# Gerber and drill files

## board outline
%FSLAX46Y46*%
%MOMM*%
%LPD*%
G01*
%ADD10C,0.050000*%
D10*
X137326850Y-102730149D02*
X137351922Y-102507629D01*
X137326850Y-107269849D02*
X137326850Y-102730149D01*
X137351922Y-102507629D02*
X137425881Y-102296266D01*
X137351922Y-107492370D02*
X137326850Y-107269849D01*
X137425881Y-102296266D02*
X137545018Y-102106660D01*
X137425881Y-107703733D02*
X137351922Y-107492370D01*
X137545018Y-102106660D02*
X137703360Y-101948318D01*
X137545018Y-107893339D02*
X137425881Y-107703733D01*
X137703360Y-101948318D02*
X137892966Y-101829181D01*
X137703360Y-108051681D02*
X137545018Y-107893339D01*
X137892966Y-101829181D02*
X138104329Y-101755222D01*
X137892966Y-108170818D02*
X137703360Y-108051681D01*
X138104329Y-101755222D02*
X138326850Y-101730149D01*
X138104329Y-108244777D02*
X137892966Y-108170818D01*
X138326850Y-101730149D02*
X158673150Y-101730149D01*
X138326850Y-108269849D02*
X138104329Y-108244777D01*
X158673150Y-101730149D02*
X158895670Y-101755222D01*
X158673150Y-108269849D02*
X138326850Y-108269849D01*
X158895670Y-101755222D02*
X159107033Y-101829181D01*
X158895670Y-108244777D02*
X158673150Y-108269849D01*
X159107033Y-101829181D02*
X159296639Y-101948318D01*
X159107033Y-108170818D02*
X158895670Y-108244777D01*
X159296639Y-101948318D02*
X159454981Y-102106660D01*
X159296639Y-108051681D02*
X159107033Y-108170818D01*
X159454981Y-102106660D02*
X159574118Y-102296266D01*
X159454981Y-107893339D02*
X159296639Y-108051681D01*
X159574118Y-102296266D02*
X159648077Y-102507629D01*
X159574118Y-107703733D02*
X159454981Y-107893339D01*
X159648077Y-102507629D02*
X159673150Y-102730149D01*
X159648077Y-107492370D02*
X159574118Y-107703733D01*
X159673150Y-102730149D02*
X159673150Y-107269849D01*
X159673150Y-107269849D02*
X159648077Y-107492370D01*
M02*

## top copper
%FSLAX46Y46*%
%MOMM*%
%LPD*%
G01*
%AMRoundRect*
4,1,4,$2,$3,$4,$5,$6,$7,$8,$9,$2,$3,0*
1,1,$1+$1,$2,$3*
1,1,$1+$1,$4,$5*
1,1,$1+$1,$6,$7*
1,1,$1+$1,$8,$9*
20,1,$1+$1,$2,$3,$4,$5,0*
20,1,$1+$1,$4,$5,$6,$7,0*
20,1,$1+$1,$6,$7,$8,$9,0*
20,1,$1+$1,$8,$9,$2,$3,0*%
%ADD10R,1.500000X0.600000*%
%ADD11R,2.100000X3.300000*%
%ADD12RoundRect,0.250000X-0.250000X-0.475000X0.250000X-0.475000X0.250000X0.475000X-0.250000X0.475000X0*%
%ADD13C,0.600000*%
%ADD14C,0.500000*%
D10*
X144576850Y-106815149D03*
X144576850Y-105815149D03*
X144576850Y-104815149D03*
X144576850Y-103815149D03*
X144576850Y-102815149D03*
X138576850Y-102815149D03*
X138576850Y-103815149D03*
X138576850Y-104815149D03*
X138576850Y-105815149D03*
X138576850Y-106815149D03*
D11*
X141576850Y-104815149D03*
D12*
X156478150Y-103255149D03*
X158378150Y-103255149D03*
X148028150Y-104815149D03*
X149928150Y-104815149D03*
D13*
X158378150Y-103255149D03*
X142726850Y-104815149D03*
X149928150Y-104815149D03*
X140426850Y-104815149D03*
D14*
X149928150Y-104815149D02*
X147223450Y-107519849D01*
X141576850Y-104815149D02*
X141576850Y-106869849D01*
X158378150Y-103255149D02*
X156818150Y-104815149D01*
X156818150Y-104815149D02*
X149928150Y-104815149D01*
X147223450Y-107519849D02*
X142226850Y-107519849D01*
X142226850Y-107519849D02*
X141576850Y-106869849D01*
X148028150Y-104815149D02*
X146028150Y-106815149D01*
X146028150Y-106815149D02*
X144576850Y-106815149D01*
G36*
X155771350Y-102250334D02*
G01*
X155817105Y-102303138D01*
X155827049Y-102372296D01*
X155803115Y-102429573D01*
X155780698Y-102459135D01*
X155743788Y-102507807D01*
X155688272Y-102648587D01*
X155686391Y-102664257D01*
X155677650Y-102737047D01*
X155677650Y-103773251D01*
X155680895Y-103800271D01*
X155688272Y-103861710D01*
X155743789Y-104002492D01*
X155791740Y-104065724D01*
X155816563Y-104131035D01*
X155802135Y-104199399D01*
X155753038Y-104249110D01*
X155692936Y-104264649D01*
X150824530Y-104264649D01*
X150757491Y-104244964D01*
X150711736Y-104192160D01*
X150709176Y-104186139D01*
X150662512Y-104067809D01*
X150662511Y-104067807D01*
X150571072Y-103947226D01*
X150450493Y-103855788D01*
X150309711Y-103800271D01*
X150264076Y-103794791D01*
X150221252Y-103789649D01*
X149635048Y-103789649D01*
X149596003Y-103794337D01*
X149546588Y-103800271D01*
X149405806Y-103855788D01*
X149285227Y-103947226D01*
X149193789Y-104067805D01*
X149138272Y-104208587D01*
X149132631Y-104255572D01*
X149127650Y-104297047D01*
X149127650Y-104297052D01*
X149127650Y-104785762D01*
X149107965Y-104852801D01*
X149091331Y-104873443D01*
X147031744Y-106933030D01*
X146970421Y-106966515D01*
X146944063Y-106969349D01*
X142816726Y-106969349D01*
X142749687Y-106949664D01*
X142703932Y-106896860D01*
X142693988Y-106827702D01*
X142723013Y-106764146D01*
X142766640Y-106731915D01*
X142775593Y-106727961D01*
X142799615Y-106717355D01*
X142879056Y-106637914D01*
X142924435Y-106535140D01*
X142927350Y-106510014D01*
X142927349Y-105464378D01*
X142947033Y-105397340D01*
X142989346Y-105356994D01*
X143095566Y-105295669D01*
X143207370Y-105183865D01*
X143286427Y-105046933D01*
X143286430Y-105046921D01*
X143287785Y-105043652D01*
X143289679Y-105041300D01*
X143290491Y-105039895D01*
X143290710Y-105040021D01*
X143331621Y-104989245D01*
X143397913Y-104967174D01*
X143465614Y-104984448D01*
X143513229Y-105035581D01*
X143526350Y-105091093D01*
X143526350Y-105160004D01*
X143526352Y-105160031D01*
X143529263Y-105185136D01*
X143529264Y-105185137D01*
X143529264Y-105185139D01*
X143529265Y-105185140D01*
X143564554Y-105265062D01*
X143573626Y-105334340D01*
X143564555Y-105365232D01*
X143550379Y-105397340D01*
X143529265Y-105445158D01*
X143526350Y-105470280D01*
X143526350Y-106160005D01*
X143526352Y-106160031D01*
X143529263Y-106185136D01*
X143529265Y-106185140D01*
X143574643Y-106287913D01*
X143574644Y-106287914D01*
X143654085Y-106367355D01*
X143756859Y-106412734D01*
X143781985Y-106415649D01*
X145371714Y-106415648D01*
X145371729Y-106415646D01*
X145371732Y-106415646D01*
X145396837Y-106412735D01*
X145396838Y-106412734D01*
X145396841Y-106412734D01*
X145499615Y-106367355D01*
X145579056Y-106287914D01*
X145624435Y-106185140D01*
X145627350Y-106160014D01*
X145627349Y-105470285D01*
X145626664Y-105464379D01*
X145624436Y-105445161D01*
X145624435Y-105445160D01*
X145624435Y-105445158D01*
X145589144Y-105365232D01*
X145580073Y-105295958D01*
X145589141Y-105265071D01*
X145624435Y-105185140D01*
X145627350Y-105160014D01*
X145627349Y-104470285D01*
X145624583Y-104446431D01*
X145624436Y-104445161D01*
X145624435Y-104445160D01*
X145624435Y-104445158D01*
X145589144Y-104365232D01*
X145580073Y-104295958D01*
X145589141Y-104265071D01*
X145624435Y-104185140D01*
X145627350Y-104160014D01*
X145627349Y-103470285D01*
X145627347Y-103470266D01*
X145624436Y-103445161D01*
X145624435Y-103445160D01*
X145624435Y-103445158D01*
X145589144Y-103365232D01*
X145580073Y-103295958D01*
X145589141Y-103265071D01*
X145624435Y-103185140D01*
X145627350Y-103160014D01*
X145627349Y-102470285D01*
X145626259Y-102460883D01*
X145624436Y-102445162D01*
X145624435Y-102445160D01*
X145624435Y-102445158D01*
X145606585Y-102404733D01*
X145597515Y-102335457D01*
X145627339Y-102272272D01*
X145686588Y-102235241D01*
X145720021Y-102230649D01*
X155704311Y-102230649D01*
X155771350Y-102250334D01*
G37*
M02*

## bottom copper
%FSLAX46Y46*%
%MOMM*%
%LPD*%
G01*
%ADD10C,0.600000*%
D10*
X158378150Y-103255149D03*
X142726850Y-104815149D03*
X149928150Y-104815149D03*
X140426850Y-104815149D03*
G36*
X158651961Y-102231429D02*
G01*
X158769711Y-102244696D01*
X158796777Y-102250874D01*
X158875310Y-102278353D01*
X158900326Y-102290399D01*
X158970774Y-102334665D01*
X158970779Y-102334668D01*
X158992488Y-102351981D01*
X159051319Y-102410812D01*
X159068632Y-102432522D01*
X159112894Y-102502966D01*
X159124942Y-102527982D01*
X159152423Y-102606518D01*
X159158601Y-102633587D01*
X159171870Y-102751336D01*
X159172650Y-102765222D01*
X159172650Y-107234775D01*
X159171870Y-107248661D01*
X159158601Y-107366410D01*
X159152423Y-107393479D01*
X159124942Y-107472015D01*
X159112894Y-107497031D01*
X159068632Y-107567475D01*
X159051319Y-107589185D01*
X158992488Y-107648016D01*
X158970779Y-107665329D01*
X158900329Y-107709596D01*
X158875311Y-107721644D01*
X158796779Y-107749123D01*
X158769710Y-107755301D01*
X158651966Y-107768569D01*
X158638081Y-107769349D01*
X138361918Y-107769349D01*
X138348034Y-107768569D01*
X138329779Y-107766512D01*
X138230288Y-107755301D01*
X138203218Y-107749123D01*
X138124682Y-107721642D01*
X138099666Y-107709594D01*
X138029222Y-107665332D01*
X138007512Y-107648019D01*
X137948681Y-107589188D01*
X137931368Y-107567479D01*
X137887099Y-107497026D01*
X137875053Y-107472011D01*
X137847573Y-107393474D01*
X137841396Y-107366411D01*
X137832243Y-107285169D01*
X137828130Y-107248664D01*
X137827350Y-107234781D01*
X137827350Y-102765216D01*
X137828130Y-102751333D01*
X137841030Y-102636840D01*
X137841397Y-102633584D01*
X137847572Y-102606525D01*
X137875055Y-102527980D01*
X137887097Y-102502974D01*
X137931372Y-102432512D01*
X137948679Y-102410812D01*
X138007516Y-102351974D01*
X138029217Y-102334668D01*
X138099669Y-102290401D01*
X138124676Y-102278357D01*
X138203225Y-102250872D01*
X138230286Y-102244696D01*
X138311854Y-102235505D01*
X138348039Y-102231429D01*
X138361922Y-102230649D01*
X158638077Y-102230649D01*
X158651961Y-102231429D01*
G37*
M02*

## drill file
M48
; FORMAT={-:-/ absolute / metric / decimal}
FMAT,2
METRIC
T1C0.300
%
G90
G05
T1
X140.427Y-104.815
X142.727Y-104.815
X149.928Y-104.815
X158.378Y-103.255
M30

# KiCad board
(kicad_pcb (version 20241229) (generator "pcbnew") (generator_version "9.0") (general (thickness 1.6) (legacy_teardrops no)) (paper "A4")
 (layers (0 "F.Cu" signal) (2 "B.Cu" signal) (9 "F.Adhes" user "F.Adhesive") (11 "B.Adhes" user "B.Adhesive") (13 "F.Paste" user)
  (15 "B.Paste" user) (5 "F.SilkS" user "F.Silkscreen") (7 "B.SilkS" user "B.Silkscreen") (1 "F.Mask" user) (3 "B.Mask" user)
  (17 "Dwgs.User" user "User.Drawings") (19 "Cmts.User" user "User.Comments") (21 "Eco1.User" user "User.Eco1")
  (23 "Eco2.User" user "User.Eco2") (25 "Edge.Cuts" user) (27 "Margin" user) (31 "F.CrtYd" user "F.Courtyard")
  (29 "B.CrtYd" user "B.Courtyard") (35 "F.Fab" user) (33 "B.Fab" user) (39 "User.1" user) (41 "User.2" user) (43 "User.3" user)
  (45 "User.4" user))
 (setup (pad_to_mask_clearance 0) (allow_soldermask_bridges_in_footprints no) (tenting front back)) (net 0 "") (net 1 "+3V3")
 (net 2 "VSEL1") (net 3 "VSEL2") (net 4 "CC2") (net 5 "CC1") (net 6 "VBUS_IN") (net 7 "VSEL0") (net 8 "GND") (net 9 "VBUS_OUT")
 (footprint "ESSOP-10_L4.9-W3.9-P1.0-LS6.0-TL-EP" (layer "F.Cu") (at 141.57685 104.815149 90)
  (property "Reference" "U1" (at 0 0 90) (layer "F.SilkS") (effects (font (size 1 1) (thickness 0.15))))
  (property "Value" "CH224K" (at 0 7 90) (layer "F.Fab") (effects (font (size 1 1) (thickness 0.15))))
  (pad "1" smd rect (at -2 3 180) (size 1.5 0.6) (layers "F.Cu" "F.Mask" "F.Paste") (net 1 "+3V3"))
  (pad "2" smd rect (at -1 3 180) (size 1.5 0.6) (layers "F.Cu" "F.Mask" "F.Paste") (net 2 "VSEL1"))
  (pad "3" smd rect (at 0 3 180) (size 1.5 0.6) (layers "F.Cu" "F.Mask" "F.Paste") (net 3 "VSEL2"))
  (pad "4" smd rect (at 1 3 180) (size 1.5 0.6) (layers "F.Cu" "F.Mask" "F.Paste"))
  (pad "5" smd rect (at 2 3 180) (size 1.5 0.6) (layers "F.Cu" "F.Mask" "F.Paste"))
  (pad "6" smd rect (at 2 -3 180) (size 1.5 0.6) (layers "F.Cu" "F.Mask" "F.Paste") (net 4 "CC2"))
  (pad "7" smd rect (at 1 -3 180) (size 1.5 0.6) (layers "F.Cu" "F.Mask" "F.Paste") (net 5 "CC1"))
  (pad "8" smd rect (at 0 -3 180) (size 1.5 0.6) (layers "F.Cu" "F.Mask" "F.Paste") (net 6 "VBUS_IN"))
  (pad "9" smd rect (at -1 -3 180) (size 1.5 0.6) (layers "F.Cu" "F.Mask" "F.Paste") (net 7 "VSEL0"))
  (pad "10" smd rect (at -2 -3 180) (size 1.5 0.6) (layers "F.Cu" "F.Mask" "F.Paste"))
  (pad "11" smd rect (at 0 0 270) (size 3.3 2.1) (layers "F.Cu" "F.Mask" "F.Paste") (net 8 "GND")))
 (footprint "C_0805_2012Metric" (layer "F.Cu") (at 157.42815 103.255149)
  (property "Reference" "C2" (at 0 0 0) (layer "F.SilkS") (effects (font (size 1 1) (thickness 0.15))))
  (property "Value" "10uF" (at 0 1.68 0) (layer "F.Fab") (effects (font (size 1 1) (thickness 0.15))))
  (pad "1" smd roundrect (at -0.95 0) (size 1 1.45) (layers "F.Cu" "F.Mask" "F.Paste") (roundrect_rratio 0.25) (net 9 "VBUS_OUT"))
  (pad "2" smd roundrect (at 0.95 0) (size 1 1.45) (layers "F.Cu" "F.Mask" "F.Paste") (roundrect_rratio 0.25) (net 8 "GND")))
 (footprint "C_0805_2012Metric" (layer "F.Cu") (at 148.97815 104.815149)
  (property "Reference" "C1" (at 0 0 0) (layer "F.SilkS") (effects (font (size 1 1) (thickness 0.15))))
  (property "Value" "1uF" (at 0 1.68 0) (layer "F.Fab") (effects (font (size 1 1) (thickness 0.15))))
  (pad "1" smd roundrect (at -0.95 0) (size 1 1.45) (layers "F.Cu" "F.Mask" "F.Paste") (roundrect_rratio 0.25) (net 1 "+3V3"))
  (pad "2" smd roundrect (at 0.95 0) (size 1 1.45) (layers "F.Cu" "F.Mask" "F.Paste") (roundrect_rratio 0.25) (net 8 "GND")))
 (gr_line (start 137.32685 102.730149) (end 137.351922 102.507629) (stroke (width 0.05) (type default)) (layer "Edge.Cuts"))
 (gr_line (start 137.32685 107.269849) (end 137.32685 102.730149) (stroke (width 0.05) (type default)) (layer "Edge.Cuts"))
 (gr_line (start 137.351922 102.507629) (end 137.425881 102.296266) (stroke (width 0.05) (type default)) (layer "Edge.Cuts"))
 (gr_line (start 137.351922 107.49237) (end 137.32685 107.269849) (stroke (width 0.05) (type default)) (layer "Edge.Cuts"))
 (gr_line (start 137.425881 102.296266) (end 137.545018 102.10666) (stroke (width 0.05) (type default)) (layer "Edge.Cuts"))
 (gr_line (start 137.425881 107.703733) (end 137.351922 107.49237) (stroke (width 0.05) (type default)) (layer "Edge.Cuts"))
 (gr_line (start 137.545018 102.10666) (end 137.70336 101.948318) (stroke (width 0.05) (type default)) (layer "Edge.Cuts"))
 (gr_line (start 137.545018 107.893339) (end 137.425881 107.703733) (stroke (width 0.05) (type default)) (layer "Edge.Cuts"))
 (gr_line (start 137.70336 101.948318) (end 137.892966 101.829181) (stroke (width 0.05) (type default)) (layer "Edge.Cuts"))
 (gr_line (start 137.70336 108.051681) (end 137.545018 107.893339) (stroke (width 0.05) (type default)) (layer "Edge.Cuts"))
 (gr_line (start 137.892966 101.829181) (end 138.104329 101.755222) (stroke (width 0.05) (type default)) (layer "Edge.Cuts"))
 (gr_line (start 137.892966 108.170818) (end 137.70336 108.051681) (stroke (width 0.05) (type default)) (layer "Edge.Cuts"))
 (gr_line (start 138.104329 101.755222) (end 138.32685 101.730149) (stroke (width 0.05) (type default)) (layer "Edge.Cuts"))
 (gr_line (start 138.104329 108.244777) (end 137.892966 108.170818) (stroke (width 0.05) (type default)) (layer "Edge.Cuts"))
 (gr_line (start 138.32685 101.730149) (end 158.67315 101.730149) (stroke (width 0.05) (type default)) (layer "Edge.Cuts"))
 (gr_line (start 138.32685 108.269849) (end 138.104329 108.244777) (stroke (width 0.05) (type default)) (layer "Edge.Cuts"))
 (gr_line (start 158.67315 101.730149) (end 158.89567 101.755222) (stroke (width 0.05) (type default)) (layer "Edge.Cuts"))
 (gr_line (start 158.67315 108.269849) (end 138.32685 108.269849) (stroke (width 0.05) (type default)) (layer "Edge.Cuts"))
 (gr_line (start 158.89567 101.755222) (end 159.107033 101.829181) (stroke (width 0.05) (type default)) (layer "Edge.Cuts"))
 (gr_line (start 158.89567 108.244777) (end 158.67315 108.269849) (stroke (width 0.05) (type default)) (layer "Edge.Cuts"))
 (gr_line (start 159.107033 101.829181) (end 159.296639 101.948318) (stroke (width 0.05) (type default)) (layer "Edge.Cuts"))
 (gr_line (start 159.107033 108.170818) (end 158.89567 108.244777) (stroke (width 0.05) (type default)) (layer "Edge.Cuts"))
 (gr_line (start 159.296639 101.948318) (end 159.454981 102.10666) (stroke (width 0.05) (type default)) (layer "Edge.Cuts"))
 (gr_line (start 159.296639 108.051681) (end 159.107033 108.170818) (stroke (width 0.05) (type default)) (layer "Edge.Cuts"))
 (gr_line (start 159.454981 102.10666) (end 159.574118 102.296266) (stroke (width 0.05) (type default)) (layer "Edge.Cuts"))
 (gr_line (start 159.454981 107.893339) (end 159.296639 108.051681) (stroke (width 0.05) (type default)) (layer "Edge.Cuts"))
 (gr_line (start 159.574118 102.296266) (end 159.648077 102.507629) (stroke (width 0.05) (type default)) (layer "Edge.Cuts"))
 (gr_line (start 159.574118 107.703733) (end 159.454981 107.893339) (stroke (width 0.05) (type default)) (layer "Edge.Cuts"))
 (gr_line (start 159.648077 102.507629) (end 159.67315 102.730149) (stroke (width 0.05) (type default)) (layer "Edge.Cuts"))
 (gr_line (start 159.648077 107.49237) (end 159.574118 107.703733) (stroke (width 0.05) (type default)) (layer "Edge.Cuts"))
 (gr_line (start 159.67315 102.730149) (end 159.67315 107.269849) (stroke (width 0.05) (type default)) (layer "Edge.Cuts"))
 (gr_line (start 159.67315 107.269849) (end 159.648077 107.49237) (stroke (width 0.05) (type default)) (layer "Edge.Cuts"))
 (segment (start 149.92815 104.815149) (end 147.22345 107.519849) (width 0.5) (layer "F.Cu") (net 8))
 (segment (start 141.57685 104.815149) (end 141.57685 106.869849) (width 0.5) (layer "F.Cu") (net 8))
 (segment (start 158.37815 103.255149) (end 156.81815 104.815149) (width 0.5) (layer "F.Cu") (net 8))
 (segment (start 156.81815 104.815149) (end 149.92815 104.815149) (width 0.5) (layer "F.Cu") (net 8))
 (segment (start 147.22345 107.519849) (end 142.22685 107.519849) (width 0.5) (layer "F.Cu") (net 8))
 (segment (start 142.22685 107.519849) (end 141.57685 106.869849) (width 0.5) (layer "F.Cu") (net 8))
 (via (at 158.37815 103.255149) (size 0.6) (drill 0.3) (layers "F.Cu" "B.Cu") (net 8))
 (via (at 142.72685 104.815149) (size 0.6) (drill 0.3) (layers "F.Cu" "B.Cu") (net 8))
 (via (at 149.92815 104.815149) (size 0.6) (drill 0.3) (layers "F.Cu" "B.Cu") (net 8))
 (via (at 140.42685 104.815149) (size 0.6) (drill 0.3) (layers "F.Cu" "B.Cu") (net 8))
 (segment (start 148.02815 104.815149) (end 146.02815 106.815149) (width 0.5) (layer "F.Cu") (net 1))
 (segment (start 146.02815 106.815149) (end 144.57685 106.815149) (width 0.5) (layer "F.Cu") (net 1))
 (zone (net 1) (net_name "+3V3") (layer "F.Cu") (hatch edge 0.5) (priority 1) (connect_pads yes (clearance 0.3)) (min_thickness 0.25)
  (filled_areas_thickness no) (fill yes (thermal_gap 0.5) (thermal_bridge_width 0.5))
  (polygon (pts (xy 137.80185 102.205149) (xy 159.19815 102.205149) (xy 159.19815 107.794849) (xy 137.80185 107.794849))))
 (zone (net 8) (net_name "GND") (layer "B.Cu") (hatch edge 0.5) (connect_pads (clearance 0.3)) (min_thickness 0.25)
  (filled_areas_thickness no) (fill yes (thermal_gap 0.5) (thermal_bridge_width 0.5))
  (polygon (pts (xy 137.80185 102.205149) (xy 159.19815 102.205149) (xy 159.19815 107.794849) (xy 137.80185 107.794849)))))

